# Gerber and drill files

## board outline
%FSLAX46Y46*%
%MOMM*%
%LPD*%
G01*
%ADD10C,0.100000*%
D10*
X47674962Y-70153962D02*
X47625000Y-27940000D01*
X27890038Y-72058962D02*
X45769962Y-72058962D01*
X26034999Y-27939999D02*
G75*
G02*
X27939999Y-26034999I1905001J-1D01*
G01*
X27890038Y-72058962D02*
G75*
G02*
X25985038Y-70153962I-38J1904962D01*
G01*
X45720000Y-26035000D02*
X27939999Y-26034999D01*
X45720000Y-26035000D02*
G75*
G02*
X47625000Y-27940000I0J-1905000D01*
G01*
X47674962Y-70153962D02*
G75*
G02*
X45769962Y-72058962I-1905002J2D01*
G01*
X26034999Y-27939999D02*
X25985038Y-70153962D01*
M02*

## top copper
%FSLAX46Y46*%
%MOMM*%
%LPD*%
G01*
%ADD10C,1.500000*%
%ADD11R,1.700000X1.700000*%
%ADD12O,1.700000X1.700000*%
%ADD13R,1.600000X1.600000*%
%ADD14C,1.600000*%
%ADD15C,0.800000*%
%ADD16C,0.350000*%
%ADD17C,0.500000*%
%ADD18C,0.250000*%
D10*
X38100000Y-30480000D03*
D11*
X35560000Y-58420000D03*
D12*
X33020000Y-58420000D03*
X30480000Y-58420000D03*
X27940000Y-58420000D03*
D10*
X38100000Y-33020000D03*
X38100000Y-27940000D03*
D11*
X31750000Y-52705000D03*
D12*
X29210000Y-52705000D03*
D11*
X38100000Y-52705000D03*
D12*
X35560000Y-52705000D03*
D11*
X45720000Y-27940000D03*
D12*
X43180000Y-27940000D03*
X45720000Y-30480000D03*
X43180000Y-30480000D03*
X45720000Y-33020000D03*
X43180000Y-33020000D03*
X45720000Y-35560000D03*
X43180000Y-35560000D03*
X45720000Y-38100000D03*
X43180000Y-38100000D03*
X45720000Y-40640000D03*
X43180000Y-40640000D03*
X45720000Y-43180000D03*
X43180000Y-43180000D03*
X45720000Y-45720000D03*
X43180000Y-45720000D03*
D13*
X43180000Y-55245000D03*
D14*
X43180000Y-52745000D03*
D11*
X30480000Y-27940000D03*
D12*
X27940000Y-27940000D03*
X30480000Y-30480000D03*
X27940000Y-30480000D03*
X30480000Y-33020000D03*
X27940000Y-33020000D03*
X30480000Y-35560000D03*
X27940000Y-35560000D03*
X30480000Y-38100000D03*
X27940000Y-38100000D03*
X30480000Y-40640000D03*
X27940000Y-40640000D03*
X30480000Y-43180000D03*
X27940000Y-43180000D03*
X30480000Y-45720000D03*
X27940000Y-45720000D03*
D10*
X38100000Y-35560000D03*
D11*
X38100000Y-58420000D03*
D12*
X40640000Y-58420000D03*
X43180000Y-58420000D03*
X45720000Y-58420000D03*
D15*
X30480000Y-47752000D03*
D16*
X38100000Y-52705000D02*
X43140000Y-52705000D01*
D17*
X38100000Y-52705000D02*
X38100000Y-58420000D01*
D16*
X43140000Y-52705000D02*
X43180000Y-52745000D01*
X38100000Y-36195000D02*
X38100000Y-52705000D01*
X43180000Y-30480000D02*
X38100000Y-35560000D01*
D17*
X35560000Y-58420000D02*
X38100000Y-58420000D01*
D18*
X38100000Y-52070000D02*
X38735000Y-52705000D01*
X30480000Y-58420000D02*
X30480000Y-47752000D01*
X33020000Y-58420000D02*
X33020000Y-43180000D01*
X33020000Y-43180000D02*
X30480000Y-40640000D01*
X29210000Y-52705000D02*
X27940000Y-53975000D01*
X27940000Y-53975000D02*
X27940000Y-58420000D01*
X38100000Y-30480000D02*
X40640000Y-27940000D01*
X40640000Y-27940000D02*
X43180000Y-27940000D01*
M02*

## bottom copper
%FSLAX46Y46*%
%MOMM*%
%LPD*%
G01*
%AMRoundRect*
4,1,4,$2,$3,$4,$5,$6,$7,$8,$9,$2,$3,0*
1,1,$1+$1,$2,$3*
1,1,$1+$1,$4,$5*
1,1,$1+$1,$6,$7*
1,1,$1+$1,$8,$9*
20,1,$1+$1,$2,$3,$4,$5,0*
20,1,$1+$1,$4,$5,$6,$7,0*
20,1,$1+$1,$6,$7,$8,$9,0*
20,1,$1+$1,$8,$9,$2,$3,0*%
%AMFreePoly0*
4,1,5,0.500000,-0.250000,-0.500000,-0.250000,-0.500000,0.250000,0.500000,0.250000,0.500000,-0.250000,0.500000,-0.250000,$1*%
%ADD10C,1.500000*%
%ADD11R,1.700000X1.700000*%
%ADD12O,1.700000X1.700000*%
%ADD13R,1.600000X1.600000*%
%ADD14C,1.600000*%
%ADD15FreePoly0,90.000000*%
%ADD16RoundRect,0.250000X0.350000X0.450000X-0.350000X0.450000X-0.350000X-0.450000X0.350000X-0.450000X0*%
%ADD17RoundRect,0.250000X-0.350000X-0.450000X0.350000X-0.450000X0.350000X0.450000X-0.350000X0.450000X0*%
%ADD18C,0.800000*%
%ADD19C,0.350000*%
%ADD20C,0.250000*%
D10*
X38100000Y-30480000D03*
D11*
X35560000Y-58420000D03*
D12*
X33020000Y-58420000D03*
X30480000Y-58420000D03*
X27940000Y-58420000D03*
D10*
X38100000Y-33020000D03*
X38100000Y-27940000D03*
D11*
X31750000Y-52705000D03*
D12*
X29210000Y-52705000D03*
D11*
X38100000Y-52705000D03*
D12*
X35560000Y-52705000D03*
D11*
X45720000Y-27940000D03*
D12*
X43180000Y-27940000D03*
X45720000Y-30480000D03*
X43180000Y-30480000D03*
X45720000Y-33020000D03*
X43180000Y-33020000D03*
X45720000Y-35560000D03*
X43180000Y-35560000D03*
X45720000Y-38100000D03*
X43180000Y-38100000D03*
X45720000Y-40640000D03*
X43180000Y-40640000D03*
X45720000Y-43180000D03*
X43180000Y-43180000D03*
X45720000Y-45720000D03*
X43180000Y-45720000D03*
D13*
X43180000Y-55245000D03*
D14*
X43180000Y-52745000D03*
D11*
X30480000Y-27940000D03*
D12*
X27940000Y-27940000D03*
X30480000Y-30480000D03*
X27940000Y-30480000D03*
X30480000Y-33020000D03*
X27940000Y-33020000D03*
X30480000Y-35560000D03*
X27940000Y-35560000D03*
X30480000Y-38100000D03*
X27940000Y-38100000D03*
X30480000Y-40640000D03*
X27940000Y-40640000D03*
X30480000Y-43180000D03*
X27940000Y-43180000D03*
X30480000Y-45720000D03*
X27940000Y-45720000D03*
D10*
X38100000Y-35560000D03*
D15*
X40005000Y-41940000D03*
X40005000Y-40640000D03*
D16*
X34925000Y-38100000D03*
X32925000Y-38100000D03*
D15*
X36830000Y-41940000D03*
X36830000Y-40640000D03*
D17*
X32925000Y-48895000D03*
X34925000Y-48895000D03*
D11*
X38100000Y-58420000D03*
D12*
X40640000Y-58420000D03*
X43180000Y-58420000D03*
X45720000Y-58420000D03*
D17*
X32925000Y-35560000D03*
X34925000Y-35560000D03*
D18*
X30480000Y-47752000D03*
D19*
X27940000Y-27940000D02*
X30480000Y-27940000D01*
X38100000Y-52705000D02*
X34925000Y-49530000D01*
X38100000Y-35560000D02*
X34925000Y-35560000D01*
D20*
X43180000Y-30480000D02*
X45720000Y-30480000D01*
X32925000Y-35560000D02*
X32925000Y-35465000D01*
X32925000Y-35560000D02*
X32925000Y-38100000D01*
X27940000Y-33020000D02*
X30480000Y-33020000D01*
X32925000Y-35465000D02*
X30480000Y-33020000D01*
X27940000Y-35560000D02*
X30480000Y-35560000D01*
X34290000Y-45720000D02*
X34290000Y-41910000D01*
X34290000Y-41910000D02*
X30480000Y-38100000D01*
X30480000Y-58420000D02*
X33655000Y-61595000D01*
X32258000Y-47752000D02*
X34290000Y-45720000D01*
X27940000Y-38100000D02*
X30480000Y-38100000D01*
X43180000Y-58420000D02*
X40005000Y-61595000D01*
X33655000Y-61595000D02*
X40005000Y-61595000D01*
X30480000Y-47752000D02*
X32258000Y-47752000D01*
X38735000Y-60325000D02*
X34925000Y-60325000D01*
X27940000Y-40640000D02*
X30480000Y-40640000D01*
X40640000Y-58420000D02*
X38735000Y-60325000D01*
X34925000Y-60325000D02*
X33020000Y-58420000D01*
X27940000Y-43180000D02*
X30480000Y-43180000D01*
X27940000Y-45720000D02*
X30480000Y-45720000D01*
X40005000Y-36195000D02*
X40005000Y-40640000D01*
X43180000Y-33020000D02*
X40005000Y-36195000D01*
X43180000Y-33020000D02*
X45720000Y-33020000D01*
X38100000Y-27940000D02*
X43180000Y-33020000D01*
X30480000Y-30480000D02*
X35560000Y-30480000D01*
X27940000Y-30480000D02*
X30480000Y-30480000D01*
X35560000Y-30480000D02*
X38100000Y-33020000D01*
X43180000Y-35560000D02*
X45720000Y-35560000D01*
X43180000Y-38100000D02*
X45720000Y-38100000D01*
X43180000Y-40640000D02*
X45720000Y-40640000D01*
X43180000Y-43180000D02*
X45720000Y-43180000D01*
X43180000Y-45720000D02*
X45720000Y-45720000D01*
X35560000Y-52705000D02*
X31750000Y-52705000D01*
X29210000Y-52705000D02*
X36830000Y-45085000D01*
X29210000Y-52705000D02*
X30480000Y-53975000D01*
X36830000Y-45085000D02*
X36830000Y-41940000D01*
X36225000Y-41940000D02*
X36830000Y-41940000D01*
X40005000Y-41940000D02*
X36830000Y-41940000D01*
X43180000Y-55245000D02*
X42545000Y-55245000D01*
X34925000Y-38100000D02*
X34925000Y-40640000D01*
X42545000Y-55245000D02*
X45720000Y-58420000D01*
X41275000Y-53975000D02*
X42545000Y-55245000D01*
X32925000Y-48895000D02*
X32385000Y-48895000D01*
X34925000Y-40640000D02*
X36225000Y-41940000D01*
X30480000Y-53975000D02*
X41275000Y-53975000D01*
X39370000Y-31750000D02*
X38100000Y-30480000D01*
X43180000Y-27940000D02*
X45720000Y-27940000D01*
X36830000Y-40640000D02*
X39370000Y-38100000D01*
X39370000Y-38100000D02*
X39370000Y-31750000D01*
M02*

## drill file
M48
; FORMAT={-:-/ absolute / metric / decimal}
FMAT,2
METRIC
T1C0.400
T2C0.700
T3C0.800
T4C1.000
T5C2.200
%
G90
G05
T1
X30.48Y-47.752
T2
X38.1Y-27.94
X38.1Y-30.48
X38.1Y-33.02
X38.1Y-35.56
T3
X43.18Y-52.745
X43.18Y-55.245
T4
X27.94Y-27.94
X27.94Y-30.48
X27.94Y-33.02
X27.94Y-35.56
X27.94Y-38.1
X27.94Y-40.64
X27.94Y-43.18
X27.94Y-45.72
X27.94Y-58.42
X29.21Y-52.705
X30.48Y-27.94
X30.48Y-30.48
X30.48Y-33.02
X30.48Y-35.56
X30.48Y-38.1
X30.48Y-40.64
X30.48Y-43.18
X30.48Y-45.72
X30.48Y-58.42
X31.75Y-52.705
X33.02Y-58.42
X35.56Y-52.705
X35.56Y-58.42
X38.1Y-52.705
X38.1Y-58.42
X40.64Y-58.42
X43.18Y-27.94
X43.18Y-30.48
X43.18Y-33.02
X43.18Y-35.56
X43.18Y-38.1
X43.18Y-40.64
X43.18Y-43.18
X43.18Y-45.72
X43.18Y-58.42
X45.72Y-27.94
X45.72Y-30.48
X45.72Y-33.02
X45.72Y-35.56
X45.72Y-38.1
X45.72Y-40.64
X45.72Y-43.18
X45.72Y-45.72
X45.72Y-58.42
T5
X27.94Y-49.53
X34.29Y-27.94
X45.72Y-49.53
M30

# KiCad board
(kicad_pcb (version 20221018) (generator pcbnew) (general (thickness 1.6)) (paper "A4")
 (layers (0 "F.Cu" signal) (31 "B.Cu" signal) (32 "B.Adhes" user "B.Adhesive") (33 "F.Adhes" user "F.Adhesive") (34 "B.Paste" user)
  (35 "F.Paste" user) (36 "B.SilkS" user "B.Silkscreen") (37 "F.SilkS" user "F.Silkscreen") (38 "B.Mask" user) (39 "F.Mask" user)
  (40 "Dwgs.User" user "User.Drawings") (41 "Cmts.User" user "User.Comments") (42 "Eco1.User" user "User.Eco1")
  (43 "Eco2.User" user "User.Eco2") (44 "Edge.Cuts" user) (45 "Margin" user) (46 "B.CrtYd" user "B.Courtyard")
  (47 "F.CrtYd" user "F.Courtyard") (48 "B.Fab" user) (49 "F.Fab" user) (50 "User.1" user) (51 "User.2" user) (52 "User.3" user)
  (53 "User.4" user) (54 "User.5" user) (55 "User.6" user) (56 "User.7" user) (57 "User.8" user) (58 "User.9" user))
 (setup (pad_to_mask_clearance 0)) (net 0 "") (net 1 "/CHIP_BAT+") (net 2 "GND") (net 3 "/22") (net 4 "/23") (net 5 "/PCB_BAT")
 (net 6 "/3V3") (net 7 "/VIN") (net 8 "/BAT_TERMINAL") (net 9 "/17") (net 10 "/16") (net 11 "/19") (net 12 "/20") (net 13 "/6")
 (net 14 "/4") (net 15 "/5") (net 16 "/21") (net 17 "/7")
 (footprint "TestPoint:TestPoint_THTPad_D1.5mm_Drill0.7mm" (layer "F.Cu") (at 38.1 30.48)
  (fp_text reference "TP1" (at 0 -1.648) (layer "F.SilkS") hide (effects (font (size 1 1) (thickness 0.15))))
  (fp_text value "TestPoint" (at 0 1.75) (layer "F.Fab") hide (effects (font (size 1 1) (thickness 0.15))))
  (pad "1" thru_hole circle (at 0 0) (size 1.5 1.5) (drill 0.7) (layers "*.Cu" "*.Mask") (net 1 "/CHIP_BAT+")))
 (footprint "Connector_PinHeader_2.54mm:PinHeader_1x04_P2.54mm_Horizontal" (layer "F.Cu") (at 35.56 58.42 -90)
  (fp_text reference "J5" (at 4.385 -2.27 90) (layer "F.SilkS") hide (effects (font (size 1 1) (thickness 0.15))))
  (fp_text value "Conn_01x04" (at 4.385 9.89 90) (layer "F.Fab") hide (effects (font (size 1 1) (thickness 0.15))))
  (pad "1" thru_hole rect (at 0 0 270) (size 1.7 1.7) (drill 1) (layers "*.Cu" "*.Mask") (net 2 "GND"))
  (pad "2" thru_hole oval (at 0 2.54 270) (size 1.7 1.7) (drill 1) (layers "*.Cu" "*.Mask") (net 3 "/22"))
  (pad "3" thru_hole oval (at 0 5.08 270) (size 1.7 1.7) (drill 1) (layers "*.Cu" "*.Mask") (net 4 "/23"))
  (pad "4" thru_hole oval (at 0 7.62 270) (size 1.7 1.7) (drill 1) (layers "*.Cu" "*.Mask") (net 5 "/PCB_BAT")))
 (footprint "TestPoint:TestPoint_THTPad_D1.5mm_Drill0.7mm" (layer "F.Cu") (at 38.1 33.02)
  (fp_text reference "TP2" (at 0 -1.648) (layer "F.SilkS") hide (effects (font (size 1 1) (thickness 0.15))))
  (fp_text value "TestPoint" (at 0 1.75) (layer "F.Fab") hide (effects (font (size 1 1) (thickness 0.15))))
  (pad "1" thru_hole circle (at 0 0) (size 1.5 1.5) (drill 0.7) (layers "*.Cu" "*.Mask") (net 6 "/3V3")))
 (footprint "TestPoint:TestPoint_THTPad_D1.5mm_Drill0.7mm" (layer "F.Cu") (at 38.1 27.94)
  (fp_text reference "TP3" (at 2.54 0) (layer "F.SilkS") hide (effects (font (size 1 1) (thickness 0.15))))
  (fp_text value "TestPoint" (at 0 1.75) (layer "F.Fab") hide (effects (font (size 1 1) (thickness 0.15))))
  (pad "1" thru_hole circle (at 0 0) (size 1.5 1.5) (drill 0.7) (layers "*.Cu" "*.Mask") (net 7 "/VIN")))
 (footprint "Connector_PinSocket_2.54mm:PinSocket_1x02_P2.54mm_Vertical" (layer "F.Cu") (at 31.75 52.705 -90)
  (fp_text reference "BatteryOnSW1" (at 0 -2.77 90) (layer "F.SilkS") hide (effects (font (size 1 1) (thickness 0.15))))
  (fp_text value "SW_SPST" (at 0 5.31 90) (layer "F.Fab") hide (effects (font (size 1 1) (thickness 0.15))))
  (pad "1" thru_hole rect (at 0 0 270) (size 1.7 1.7) (drill 1) (layers "*.Cu" "*.Mask") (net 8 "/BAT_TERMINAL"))
  (pad "2" thru_hole oval (at 0 2.54 270) (size 1.7 1.7) (drill 1) (layers "*.Cu" "*.Mask") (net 5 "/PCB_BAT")))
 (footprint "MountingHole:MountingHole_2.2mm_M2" (layer "F.Cu") (at 45.72 49.53)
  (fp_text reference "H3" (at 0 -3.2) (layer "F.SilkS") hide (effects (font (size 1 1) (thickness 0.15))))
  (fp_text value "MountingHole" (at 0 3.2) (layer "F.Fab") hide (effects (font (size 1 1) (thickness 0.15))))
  (pad "" np_thru_hole circle (at 0 0) (size 2.2 2.2) (drill 2.2) (layers "*.Cu" "*.Mask")))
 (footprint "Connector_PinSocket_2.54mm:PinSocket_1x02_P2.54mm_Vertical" (layer "F.Cu") (at 38.1 52.705 -90)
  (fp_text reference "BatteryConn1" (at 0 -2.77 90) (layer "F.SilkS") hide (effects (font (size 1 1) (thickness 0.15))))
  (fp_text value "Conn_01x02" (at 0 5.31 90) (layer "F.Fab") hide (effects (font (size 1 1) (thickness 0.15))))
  (pad "1" thru_hole rect (at 0 0 270) (size 1.7 1.7) (drill 1) (layers "*.Cu" "*.Mask") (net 2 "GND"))
  (pad "2" thru_hole oval (at 0 2.54 270) (size 1.7 1.7) (drill 1) (layers "*.Cu" "*.Mask") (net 8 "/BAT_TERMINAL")))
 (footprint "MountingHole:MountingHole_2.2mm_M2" (layer "F.Cu") (at 34.29 27.94)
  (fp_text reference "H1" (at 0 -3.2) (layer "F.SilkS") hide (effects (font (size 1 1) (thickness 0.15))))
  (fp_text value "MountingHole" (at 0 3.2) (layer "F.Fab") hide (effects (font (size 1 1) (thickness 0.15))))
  (pad "" np_thru_hole circle (at 0 0) (size 2.2 2.2) (drill 2.2) (layers "*.Cu" "*.Mask")))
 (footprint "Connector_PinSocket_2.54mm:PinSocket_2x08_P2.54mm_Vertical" (layer "F.Cu") (at 45.72 27.94)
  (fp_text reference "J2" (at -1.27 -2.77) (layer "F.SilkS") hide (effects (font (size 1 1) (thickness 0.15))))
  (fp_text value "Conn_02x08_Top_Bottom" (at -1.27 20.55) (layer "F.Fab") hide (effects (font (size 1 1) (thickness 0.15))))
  (pad "1" thru_hole rect (at 0 0) (size 1.7 1.7) (drill 1) (layers "*.Cu" "*.Mask") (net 1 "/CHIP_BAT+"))
  (pad "2" thru_hole oval (at -2.54 0) (size 1.7 1.7) (drill 1) (layers "*.Cu" "*.Mask") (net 1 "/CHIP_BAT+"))
  (pad "3" thru_hole oval (at 0 2.54) (size 1.7 1.7) (drill 1) (layers "*.Cu" "*.Mask") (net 2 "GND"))
  (pad "4" thru_hole oval (at -2.54 2.54) (size 1.7 1.7) (drill 1) (layers "*.Cu" "*.Mask") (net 2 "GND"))
  (pad "5" thru_hole oval (at 0 5.08) (size 1.7 1.7) (drill 1) (layers "*.Cu" "*.Mask") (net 7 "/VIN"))
  (pad "6" thru_hole oval (at -2.54 5.08) (size 1.7 1.7) (drill 1) (layers "*.Cu" "*.Mask") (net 7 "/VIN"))
  (pad "7" thru_hole oval (at 0 7.62) (size 1.7 1.7) (drill 1) (layers "*.Cu" "*.Mask") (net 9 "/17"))
  (pad "8" thru_hole oval (at -2.54 7.62) (size 1.7 1.7) (drill 1) (layers "*.Cu" "*.Mask") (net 9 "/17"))
  (pad "9" thru_hole oval (at 0 10.16) (size 1.7 1.7) (drill 1) (layers "*.Cu" "*.Mask") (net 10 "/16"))
  (pad "10" thru_hole oval (at -2.54 10.16) (size 1.7 1.7) (drill 1) (layers "*.Cu" "*.Mask") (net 10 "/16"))
  (pad "11" thru_hole oval (at 0 12.7) (size 1.7 1.7) (drill 1) (layers "*.Cu" "*.Mask") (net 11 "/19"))
  (pad "12" thru_hole oval (at -2.54 12.7) (size 1.7 1.7) (drill 1) (layers "*.Cu" "*.Mask") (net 11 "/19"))
  (pad "13" thru_hole oval (at 0 15.24) (size 1.7 1.7) (drill 1) (layers "*.Cu" "*.Mask") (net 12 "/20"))
  (pad "14" thru_hole oval (at -2.54 15.24) (size 1.7 1.7) (drill 1) (layers "*.Cu" "*.Mask") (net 12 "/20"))
  (pad "15" thru_hole oval (at 0 17.78) (size 1.7 1.7) (drill 1) (layers "*.Cu" "*.Mask") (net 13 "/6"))
  (pad "16" thru_hole oval (at -2.54 17.78) (size 1.7 1.7) (drill 1) (layers "*.Cu" "*.Mask") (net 13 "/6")))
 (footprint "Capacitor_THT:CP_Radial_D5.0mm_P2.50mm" (layer "F.Cu") (at 43.18 55.245 90)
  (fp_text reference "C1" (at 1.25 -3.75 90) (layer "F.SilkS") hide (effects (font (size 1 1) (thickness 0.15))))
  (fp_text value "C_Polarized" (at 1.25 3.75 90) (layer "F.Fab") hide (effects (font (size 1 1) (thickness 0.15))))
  (pad "1" thru_hole rect (at 0 0 90) (size 1.6 1.6) (drill 0.8) (layers "*.Cu" "*.Mask") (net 5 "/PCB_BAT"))
  (pad "2" thru_hole circle (at 2.5 0 90) (size 1.6 1.6) (drill 0.8) (layers "*.Cu" "*.Mask") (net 2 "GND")))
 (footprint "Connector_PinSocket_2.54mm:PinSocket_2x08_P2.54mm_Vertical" (layer "F.Cu") (at 30.48 27.94)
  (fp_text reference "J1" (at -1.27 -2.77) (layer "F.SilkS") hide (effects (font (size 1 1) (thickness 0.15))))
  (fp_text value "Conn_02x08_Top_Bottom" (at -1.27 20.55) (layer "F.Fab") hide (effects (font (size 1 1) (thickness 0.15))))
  (pad "1" thru_hole rect (at 0 0) (size 1.7 1.7) (drill 1) (layers "*.Cu" "*.Mask") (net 2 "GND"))
  (pad "2" thru_hole oval (at -2.54 0) (size 1.7 1.7) (drill 1) (layers "*.Cu" "*.Mask") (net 2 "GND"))
  (pad "3" thru_hole oval (at 0 2.54) (size 1.7 1.7) (drill 1) (layers "*.Cu" "*.Mask") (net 6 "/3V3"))
  (pad "4" thru_hole oval (at -2.54 2.54) (size 1.7 1.7) (drill 1) (layers "*.Cu" "*.Mask") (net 6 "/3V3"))
  (pad "5" thru_hole oval (at 0 5.08) (size 1.7 1.7) (drill 1) (layers "*.Cu" "*.Mask") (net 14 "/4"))
  (pad "6" thru_hole oval (at -2.54 5.08) (size 1.7 1.7) (drill 1) (layers "*.Cu" "*.Mask") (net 14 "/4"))
  (pad "7" thru_hole oval (at 0 7.62) (size 1.7 1.7) (drill 1) (layers "*.Cu" "*.Mask") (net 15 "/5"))
  (pad "8" thru_hole oval (at -2.54 7.62) (size 1.7 1.7) (drill 1) (layers "*.Cu" "*.Mask") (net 15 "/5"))
  (pad "9" thru_hole oval (at 0 10.16) (size 1.7 1.7) (drill 1) (layers "*.Cu" "*.Mask") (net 4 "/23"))
  (pad "10" thru_hole oval (at -2.54 10.16) (size 1.7 1.7) (drill 1) (layers "*.Cu" "*.Mask") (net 4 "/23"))
  (pad "11" thru_hole oval (at 0 12.7) (size 1.7 1.7) (drill 1) (layers "*.Cu" "*.Mask") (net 3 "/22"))
  (pad "12" thru_hole oval (at -2.54 12.7) (size 1.7 1.7) (drill 1) (layers "*.Cu" "*.Mask") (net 3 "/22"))
  (pad "13" thru_hole oval (at 0 15.24) (size 1.7 1.7) (drill 1) (layers "*.Cu" "*.Mask") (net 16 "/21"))
  (pad "14" thru_hole oval (at -2.54 15.24) (size 1.7 1.7) (drill 1) (layers "*.Cu" "*.Mask") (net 16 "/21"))
  (pad "15" thru_hole oval (at 0 17.78) (size 1.7 1.7) (drill 1) (layers "*.Cu" "*.Mask") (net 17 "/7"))
  (pad "16" thru_hole oval (at -2.54 17.78) (size 1.7 1.7) (drill 1) (layers "*.Cu" "*.Mask") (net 17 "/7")))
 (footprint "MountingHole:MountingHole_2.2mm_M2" (layer "F.Cu") (at 27.94 49.53)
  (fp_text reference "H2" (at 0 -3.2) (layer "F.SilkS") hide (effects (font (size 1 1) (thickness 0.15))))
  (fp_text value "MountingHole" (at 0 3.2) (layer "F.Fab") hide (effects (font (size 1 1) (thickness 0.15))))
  (pad "" np_thru_hole circle (at 0 0) (size 2.2 2.2) (drill 2.2) (layers "*.Cu" "*.Mask")))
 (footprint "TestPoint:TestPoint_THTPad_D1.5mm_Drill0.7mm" (layer "F.Cu") (at 38.1 35.56)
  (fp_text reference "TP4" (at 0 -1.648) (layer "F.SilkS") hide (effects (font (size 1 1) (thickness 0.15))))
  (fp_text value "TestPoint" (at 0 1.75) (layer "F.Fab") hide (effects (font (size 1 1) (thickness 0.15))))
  (pad "1" thru_hole circle (at 0 0) (size 1.5 1.5) (drill 0.7) (layers "*.Cu" "*.Mask") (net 2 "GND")))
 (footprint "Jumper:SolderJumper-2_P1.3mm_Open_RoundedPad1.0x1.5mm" (layer "B.Cu") (at 40.005 41.29 90) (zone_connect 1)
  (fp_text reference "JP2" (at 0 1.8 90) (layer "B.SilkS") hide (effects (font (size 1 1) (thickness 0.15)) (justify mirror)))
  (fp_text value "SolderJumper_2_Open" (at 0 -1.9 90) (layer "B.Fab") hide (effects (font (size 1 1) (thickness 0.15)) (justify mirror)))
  (pad "1" smd custom (at -0.65 0 90) (size 1 0.5) (layers "B.Cu" "B.Mask") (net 5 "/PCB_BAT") (zone_connect 2) (thermal_bridge_angle 45)
   (options (clearance outline) (anchor rect)) (primitives))
  (pad "2" smd custom (at 0.65 0 90) (size 1 0.5) (layers "B.Cu" "B.Mask") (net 7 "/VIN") (zone_connect 2) (thermal_bridge_angle 45)
   (options (clearance outline) (anchor rect)) (primitives)))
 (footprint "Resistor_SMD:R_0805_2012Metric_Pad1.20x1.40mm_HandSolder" (layer "B.Cu") (at 33.925 38.1 180)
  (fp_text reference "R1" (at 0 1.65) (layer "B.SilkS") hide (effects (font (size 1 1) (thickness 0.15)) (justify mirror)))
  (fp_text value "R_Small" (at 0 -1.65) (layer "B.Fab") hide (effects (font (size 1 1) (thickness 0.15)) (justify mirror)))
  (pad "1" smd roundrect (at -1 0 180) (size 1.2 1.4) (layers "B.Cu" "B.Paste" "B.Mask") (roundrect_rratio 0.2083333333) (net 5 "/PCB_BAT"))
  (pad "2" smd roundrect (at 1 0 180) (size 1.2 1.4) (layers "B.Cu" "B.Paste" "B.Mask") (roundrect_rratio 0.2083333333) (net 14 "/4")))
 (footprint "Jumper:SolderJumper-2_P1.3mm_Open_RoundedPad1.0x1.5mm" (layer "B.Cu") (at 36.83 41.29 90) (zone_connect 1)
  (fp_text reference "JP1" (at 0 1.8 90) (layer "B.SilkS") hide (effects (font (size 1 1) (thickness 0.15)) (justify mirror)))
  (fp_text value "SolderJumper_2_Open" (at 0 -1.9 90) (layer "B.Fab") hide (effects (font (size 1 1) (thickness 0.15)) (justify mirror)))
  (pad "1" smd custom (at -0.65 0 90) (size 1 0.5) (layers "B.Cu" "B.Mask") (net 5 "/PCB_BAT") (zone_connect 2) (thermal_bridge_angle 45)
   (options (clearance outline) (anchor rect)) (primitives))
  (pad "2" smd custom (at 0.65 0 90) (size 1 0.5) (layers "B.Cu" "B.Mask") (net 1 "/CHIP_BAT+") (zone_connect 2) (thermal_bridge_angle 45)
   (options (clearance outline) (anchor rect)) (primitives)))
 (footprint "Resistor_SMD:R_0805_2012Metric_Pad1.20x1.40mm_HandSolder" (layer "B.Cu") (at 33.925 48.895)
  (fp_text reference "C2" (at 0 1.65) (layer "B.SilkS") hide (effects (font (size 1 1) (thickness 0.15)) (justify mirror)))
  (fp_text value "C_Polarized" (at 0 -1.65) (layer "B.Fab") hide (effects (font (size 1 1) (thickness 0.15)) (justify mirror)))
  (pad "1" smd roundrect (at -1 0) (size 1.2 1.4) (layers "B.Cu" "B.Paste" "B.Mask") (roundrect_rratio 0.2083333333) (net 5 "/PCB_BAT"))
  (pad "2" smd roundrect (at 1 0) (size 1.2 1.4) (layers "B.Cu" "B.Paste" "B.Mask") (roundrect_rratio 0.2083333333) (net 2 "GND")))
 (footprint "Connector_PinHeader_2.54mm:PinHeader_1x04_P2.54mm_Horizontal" (layer "B.Cu") (at 38.1 58.42 -90)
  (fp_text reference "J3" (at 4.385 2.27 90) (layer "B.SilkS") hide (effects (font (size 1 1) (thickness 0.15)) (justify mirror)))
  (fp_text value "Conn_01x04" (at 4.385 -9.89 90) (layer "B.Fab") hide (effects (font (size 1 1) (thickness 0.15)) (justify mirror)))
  (pad "1" thru_hole rect (at 0 0 270) (size 1.7 1.7) (drill 1) (layers "*.Cu" "*.Mask") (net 2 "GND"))
  (pad "2" thru_hole oval (at 0 -2.54 270) (size 1.7 1.7) (drill 1) (layers "*.Cu" "*.Mask") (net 3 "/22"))
  (pad "3" thru_hole oval (at 0 -5.08 270) (size 1.7 1.7) (drill 1) (layers "*.Cu" "*.Mask") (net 4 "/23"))
  (pad "4" thru_hole oval (at 0 -7.62 270) (size 1.7 1.7) (drill 1) (layers "*.Cu" "*.Mask") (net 5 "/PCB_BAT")))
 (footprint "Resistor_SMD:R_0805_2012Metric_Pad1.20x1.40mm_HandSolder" (layer "B.Cu") (at 33.925 35.56)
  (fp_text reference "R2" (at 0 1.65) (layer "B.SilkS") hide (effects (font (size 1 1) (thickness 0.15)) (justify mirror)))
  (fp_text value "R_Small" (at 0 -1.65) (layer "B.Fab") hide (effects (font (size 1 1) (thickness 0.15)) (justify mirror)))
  (pad "1" smd roundrect (at -1 0) (size 1.2 1.4) (layers "B.Cu" "B.Paste" "B.Mask") (roundrect_rratio 0.2083333333) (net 14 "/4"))
  (pad "2" smd roundrect (at 1 0) (size 1.2 1.4) (layers "B.Cu" "B.Paste" "B.Mask") (roundrect_rratio 0.2083333333) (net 2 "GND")))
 (gr_line (start 47.674962 70.153962) (end 47.625 27.94) (stroke (width 0.1) (type default)) (layer "Edge.Cuts"))
 (gr_line (start 27.890038 72.058962) (end 45.769962 72.058962) (stroke (width 0.1) (type default)) (layer "Edge.Cuts"))
 (gr_arc (start 26.034999 27.939999) (mid 26.592961 26.592961) (end 27.939999 26.034999) (stroke (width 0.1) (type default))
  (layer "Edge.Cuts"))
 (gr_arc (start 27.890038 72.058962) (mid 26.543 71.501) (end 25.985038 70.153962) (stroke (width 0.1) (type default)) (layer "Edge.Cuts"))
 (gr_line (start 45.72 26.035) (end 27.939999 26.034999) (stroke (width 0.1) (type default)) (layer "Edge.Cuts"))
 (gr_arc (start 45.72 26.035) (mid 47.067038 26.592962) (end 47.625 27.94) (stroke (width 0.1) (type default)) (layer "Edge.Cuts"))
 (gr_arc (start 47.674962 70.153962) (mid 47.117 71.501) (end 45.769962 72.058962) (stroke (width 0.1) (type default)) (layer "Edge.Cuts"))
 (gr_line (start 26.034999 27.939999) (end 25.985038 70.153962) (stroke (width 0.1) (type default)) (layer "Edge.Cuts"))
 (segment (start 38.1 52.705) (end 43.14 52.705) (width 0.35) (layer "F.Cu") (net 2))
 (segment (start 38.1 52.705) (end 38.1 58.42) (width 0.5) (layer "F.Cu") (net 2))
 (segment (start 43.14 52.705) (end 43.18 52.745) (width 0.35) (layer "F.Cu") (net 2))
 (segment (start 38.1 36.195) (end 38.1 52.705) (width 0.35) (layer "F.Cu") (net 2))
 (segment (start 43.18 30.48) (end 38.1 35.56) (width 0.35) (layer "F.Cu") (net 2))
 (segment (start 35.56 58.42) (end 38.1 58.42) (width 0.5) (layer "F.Cu") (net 2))
 (segment (start 38.1 52.07) (end 38.735 52.705) (width 0.25) (layer "F.Cu") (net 2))
 (segment (start 27.94 27.94) (end 30.48 27.94) (width 0.35) (layer "B.Cu") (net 2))
 (segment (start 38.1 52.705) (end 34.925 49.53) (width 0.35) (layer "B.Cu") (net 2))
 (segment (start 38.1 35.56) (end 34.925 35.56) (width 0.35) (layer "B.Cu") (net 2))
 (segment (start 43.18 30.48) (end 45.72 30.48) (width 0.25) (layer "B.Cu") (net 2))
 (segment (start 32.925 35.56) (end 32.925 35.465) (width 0.25) (layer "B.Cu") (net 14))
 (segment (start 32.925 35.56) (end 32.925 38.1) (width 0.25) (layer "B.Cu") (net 14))
 (segment (start 27.94 33.02) (end 30.48 33.02) (width 0.25) (layer "B.Cu") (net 14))
 (segment (start 32.925 35.465) (end 30.48 33.02) (width 0.25) (layer "B.Cu") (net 14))
 (segment (start 27.94 35.56) (end 30.48 35.56) (width 0.25) (layer "B.Cu") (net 15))
 (segment (start 30.48 58.42) (end 30.48 47.752) (width 0.25) (layer "F.Cu") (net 4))
 (via (at 30.48 47.752) (size 0.8) (drill 0.4) (layers "F.Cu" "B.Cu") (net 4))
 (segment (start 34.29 45.72) (end 34.29 41.91) (width 0.25) (layer "B.Cu") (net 4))
 (segment (start 34.29 41.91) (end 30.48 38.1) (width 0.25) (layer "B.Cu") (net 4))
 (segment (start 30.48 58.42) (end 33.655 61.595) (width 0.25) (layer "B.Cu") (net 4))
 (segment (start 32.258 47.752) (end 34.29 45.72) (width 0.25) (layer "B.Cu") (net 4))
 (segment (start 27.94 38.1) (end 30.48 38.1) (width 0.25) (layer "B.Cu") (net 4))
 (segment (start 43.18 58.42) (end 40.005 61.595) (width 0.25) (layer "B.Cu") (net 4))
 (segment (start 33.655 61.595) (end 40.005 61.595) (width 0.25) (layer "B.Cu") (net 4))
 (segment (start 30.48 47.752) (end 32.258 47.752) (width 0.25) (layer "B.Cu") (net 4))
 (segment (start 33.02 58.42) (end 33.02 43.18) (width 0.25) (layer "F.Cu") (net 3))
 (segment (start 33.02 43.18) (end 30.48 40.64) (width 0.25) (layer "F.Cu") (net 3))
 (segment (start 38.735 60.325) (end 34.925 60.325) (width 0.25) (layer "B.Cu") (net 3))
 (segment (start 27.94 40.64) (end 30.48 40.64) (width 0.25) (layer "B.Cu") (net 3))
 (segment (start 40.64 58.42) (end 38.735 60.325) (width 0.25) (layer "B.Cu") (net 3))
 (segment (start 34.925 60.325) (end 33.02 58.42) (width 0.25) (layer "B.Cu") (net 3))
 (segment (start 27.94 43.18) (end 30.48 43.18) (width 0.25) (layer "B.Cu") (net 16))
 (segment (start 27.94 45.72) (end 30.48 45.72) (width 0.25) (layer "B.Cu") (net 17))
 (segment (start 40.005 36.195) (end 40.005 40.64) (width 0.25) (layer "B.Cu") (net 7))
 (segment (start 43.18 33.02) (end 40.005 36.195) (width 0.25) (layer "B.Cu") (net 7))
 (segment (start 43.18 33.02) (end 45.72 33.02) (width 0.25) (layer "B.Cu") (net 7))
 (segment (start 38.1 27.94) (end 43.18 33.02) (width 0.25) (layer "B.Cu") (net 7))
 (segment (start 30.48 30.48) (end 35.56 30.48) (width 0.25) (layer "B.Cu") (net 6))
 (segment (start 27.94 30.48) (end 30.48 30.48) (width 0.25) (layer "B.Cu") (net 6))
 (segment (start 35.56 30.48) (end 38.1 33.02) (width 0.25) (layer "B.Cu") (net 6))
 (segment (start 43.18 35.56) (end 45.72 35.56) (width 0.25) (layer "B.Cu") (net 9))
 (segment (start 43.18 38.1) (end 45.72 38.1) (width 0.25) (layer "B.Cu") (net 10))
 (segment (start 43.18 40.64) (end 45.72 40.64) (width 0.25) (layer "B.Cu") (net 11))
 (segment (start 43.18 43.18) (end 45.72 43.18) (width 0.25) (layer "B.Cu") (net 12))
 (segment (start 43.18 45.72) (end 45.72 45.72) (width 0.25) (layer "B.Cu") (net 13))
 (segment (start 35.56 52.705) (end 31.75 52.705) (width 0.25) (layer "B.Cu") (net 8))
 (segment (start 29.21 52.705) (end 27.94 53.975) (width 0.25) (layer "F.Cu") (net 5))
 (segment (start 27.94 53.975) (end 27.94 58.42) (width 0.25) (layer "F.Cu") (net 5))
 (segment (start 29.21 52.705) (end 36.83 45.085) (width 0.25) (layer "B.Cu") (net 5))
 (segment (start 29.21 52.705) (end 30.48 53.975) (width 0.25) (layer "B.Cu") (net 5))
 (segment (start 36.83 45.085) (end 36.83 41.94) (width 0.25) (layer "B.Cu") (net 5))
 (segment (start 36.225 41.94) (end 36.83 41.94) (width 0.25) (layer "B.Cu") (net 5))
 (segment (start 40.005 41.94) (end 36.83 41.94) (width 0.25) (layer "B.Cu") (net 5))
 (segment (start 43.18 55.245) (end 42.545 55.245) (width 0.25) (layer "B.Cu") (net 5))
 (segment (start 34.925 38.1) (end 34.925 40.64) (width 0.25) (layer "B.Cu") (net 5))
 (segment (start 42.545 55.245) (end 45.72 58.42) (width 0.25) (layer "B.Cu") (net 5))
 (segment (start 41.275 53.975) (end 42.545 55.245) (width 0.25) (layer "B.Cu") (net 5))
 (segment (start 32.925 48.895) (end 32.385 48.895) (width 0.25) (layer "B.Cu") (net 5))
 (segment (start 34.925 40.64) (end 36.225 41.94) (width 0.25) (layer "B.Cu") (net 5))
 (segment (start 30.48 53.975) (end 41.275 53.975) (width 0.25) (layer "B.Cu") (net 5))
 (segment (start 38.1 30.48) (end 40.64 27.94) (width 0.25) (layer "F.Cu") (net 1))
 (segment (start 40.64 27.94) (end 43.18 27.94) (width 0.25) (layer "F.Cu") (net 1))
 (segment (start 39.37 31.75) (end 38.1 30.48) (width 0.25) (layer "B.Cu") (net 1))
 (segment (start 43.18 27.94) (end 45.72 27.94) (width 0.25) (layer "B.Cu") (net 1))
 (segment (start 36.83 40.64) (end 39.37 38.1) (width 0.25) (layer "B.Cu") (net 1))
 (segment (start 39.37 38.1) (end 39.37 31.75) (width 0.25) (layer "B.Cu") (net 1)))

